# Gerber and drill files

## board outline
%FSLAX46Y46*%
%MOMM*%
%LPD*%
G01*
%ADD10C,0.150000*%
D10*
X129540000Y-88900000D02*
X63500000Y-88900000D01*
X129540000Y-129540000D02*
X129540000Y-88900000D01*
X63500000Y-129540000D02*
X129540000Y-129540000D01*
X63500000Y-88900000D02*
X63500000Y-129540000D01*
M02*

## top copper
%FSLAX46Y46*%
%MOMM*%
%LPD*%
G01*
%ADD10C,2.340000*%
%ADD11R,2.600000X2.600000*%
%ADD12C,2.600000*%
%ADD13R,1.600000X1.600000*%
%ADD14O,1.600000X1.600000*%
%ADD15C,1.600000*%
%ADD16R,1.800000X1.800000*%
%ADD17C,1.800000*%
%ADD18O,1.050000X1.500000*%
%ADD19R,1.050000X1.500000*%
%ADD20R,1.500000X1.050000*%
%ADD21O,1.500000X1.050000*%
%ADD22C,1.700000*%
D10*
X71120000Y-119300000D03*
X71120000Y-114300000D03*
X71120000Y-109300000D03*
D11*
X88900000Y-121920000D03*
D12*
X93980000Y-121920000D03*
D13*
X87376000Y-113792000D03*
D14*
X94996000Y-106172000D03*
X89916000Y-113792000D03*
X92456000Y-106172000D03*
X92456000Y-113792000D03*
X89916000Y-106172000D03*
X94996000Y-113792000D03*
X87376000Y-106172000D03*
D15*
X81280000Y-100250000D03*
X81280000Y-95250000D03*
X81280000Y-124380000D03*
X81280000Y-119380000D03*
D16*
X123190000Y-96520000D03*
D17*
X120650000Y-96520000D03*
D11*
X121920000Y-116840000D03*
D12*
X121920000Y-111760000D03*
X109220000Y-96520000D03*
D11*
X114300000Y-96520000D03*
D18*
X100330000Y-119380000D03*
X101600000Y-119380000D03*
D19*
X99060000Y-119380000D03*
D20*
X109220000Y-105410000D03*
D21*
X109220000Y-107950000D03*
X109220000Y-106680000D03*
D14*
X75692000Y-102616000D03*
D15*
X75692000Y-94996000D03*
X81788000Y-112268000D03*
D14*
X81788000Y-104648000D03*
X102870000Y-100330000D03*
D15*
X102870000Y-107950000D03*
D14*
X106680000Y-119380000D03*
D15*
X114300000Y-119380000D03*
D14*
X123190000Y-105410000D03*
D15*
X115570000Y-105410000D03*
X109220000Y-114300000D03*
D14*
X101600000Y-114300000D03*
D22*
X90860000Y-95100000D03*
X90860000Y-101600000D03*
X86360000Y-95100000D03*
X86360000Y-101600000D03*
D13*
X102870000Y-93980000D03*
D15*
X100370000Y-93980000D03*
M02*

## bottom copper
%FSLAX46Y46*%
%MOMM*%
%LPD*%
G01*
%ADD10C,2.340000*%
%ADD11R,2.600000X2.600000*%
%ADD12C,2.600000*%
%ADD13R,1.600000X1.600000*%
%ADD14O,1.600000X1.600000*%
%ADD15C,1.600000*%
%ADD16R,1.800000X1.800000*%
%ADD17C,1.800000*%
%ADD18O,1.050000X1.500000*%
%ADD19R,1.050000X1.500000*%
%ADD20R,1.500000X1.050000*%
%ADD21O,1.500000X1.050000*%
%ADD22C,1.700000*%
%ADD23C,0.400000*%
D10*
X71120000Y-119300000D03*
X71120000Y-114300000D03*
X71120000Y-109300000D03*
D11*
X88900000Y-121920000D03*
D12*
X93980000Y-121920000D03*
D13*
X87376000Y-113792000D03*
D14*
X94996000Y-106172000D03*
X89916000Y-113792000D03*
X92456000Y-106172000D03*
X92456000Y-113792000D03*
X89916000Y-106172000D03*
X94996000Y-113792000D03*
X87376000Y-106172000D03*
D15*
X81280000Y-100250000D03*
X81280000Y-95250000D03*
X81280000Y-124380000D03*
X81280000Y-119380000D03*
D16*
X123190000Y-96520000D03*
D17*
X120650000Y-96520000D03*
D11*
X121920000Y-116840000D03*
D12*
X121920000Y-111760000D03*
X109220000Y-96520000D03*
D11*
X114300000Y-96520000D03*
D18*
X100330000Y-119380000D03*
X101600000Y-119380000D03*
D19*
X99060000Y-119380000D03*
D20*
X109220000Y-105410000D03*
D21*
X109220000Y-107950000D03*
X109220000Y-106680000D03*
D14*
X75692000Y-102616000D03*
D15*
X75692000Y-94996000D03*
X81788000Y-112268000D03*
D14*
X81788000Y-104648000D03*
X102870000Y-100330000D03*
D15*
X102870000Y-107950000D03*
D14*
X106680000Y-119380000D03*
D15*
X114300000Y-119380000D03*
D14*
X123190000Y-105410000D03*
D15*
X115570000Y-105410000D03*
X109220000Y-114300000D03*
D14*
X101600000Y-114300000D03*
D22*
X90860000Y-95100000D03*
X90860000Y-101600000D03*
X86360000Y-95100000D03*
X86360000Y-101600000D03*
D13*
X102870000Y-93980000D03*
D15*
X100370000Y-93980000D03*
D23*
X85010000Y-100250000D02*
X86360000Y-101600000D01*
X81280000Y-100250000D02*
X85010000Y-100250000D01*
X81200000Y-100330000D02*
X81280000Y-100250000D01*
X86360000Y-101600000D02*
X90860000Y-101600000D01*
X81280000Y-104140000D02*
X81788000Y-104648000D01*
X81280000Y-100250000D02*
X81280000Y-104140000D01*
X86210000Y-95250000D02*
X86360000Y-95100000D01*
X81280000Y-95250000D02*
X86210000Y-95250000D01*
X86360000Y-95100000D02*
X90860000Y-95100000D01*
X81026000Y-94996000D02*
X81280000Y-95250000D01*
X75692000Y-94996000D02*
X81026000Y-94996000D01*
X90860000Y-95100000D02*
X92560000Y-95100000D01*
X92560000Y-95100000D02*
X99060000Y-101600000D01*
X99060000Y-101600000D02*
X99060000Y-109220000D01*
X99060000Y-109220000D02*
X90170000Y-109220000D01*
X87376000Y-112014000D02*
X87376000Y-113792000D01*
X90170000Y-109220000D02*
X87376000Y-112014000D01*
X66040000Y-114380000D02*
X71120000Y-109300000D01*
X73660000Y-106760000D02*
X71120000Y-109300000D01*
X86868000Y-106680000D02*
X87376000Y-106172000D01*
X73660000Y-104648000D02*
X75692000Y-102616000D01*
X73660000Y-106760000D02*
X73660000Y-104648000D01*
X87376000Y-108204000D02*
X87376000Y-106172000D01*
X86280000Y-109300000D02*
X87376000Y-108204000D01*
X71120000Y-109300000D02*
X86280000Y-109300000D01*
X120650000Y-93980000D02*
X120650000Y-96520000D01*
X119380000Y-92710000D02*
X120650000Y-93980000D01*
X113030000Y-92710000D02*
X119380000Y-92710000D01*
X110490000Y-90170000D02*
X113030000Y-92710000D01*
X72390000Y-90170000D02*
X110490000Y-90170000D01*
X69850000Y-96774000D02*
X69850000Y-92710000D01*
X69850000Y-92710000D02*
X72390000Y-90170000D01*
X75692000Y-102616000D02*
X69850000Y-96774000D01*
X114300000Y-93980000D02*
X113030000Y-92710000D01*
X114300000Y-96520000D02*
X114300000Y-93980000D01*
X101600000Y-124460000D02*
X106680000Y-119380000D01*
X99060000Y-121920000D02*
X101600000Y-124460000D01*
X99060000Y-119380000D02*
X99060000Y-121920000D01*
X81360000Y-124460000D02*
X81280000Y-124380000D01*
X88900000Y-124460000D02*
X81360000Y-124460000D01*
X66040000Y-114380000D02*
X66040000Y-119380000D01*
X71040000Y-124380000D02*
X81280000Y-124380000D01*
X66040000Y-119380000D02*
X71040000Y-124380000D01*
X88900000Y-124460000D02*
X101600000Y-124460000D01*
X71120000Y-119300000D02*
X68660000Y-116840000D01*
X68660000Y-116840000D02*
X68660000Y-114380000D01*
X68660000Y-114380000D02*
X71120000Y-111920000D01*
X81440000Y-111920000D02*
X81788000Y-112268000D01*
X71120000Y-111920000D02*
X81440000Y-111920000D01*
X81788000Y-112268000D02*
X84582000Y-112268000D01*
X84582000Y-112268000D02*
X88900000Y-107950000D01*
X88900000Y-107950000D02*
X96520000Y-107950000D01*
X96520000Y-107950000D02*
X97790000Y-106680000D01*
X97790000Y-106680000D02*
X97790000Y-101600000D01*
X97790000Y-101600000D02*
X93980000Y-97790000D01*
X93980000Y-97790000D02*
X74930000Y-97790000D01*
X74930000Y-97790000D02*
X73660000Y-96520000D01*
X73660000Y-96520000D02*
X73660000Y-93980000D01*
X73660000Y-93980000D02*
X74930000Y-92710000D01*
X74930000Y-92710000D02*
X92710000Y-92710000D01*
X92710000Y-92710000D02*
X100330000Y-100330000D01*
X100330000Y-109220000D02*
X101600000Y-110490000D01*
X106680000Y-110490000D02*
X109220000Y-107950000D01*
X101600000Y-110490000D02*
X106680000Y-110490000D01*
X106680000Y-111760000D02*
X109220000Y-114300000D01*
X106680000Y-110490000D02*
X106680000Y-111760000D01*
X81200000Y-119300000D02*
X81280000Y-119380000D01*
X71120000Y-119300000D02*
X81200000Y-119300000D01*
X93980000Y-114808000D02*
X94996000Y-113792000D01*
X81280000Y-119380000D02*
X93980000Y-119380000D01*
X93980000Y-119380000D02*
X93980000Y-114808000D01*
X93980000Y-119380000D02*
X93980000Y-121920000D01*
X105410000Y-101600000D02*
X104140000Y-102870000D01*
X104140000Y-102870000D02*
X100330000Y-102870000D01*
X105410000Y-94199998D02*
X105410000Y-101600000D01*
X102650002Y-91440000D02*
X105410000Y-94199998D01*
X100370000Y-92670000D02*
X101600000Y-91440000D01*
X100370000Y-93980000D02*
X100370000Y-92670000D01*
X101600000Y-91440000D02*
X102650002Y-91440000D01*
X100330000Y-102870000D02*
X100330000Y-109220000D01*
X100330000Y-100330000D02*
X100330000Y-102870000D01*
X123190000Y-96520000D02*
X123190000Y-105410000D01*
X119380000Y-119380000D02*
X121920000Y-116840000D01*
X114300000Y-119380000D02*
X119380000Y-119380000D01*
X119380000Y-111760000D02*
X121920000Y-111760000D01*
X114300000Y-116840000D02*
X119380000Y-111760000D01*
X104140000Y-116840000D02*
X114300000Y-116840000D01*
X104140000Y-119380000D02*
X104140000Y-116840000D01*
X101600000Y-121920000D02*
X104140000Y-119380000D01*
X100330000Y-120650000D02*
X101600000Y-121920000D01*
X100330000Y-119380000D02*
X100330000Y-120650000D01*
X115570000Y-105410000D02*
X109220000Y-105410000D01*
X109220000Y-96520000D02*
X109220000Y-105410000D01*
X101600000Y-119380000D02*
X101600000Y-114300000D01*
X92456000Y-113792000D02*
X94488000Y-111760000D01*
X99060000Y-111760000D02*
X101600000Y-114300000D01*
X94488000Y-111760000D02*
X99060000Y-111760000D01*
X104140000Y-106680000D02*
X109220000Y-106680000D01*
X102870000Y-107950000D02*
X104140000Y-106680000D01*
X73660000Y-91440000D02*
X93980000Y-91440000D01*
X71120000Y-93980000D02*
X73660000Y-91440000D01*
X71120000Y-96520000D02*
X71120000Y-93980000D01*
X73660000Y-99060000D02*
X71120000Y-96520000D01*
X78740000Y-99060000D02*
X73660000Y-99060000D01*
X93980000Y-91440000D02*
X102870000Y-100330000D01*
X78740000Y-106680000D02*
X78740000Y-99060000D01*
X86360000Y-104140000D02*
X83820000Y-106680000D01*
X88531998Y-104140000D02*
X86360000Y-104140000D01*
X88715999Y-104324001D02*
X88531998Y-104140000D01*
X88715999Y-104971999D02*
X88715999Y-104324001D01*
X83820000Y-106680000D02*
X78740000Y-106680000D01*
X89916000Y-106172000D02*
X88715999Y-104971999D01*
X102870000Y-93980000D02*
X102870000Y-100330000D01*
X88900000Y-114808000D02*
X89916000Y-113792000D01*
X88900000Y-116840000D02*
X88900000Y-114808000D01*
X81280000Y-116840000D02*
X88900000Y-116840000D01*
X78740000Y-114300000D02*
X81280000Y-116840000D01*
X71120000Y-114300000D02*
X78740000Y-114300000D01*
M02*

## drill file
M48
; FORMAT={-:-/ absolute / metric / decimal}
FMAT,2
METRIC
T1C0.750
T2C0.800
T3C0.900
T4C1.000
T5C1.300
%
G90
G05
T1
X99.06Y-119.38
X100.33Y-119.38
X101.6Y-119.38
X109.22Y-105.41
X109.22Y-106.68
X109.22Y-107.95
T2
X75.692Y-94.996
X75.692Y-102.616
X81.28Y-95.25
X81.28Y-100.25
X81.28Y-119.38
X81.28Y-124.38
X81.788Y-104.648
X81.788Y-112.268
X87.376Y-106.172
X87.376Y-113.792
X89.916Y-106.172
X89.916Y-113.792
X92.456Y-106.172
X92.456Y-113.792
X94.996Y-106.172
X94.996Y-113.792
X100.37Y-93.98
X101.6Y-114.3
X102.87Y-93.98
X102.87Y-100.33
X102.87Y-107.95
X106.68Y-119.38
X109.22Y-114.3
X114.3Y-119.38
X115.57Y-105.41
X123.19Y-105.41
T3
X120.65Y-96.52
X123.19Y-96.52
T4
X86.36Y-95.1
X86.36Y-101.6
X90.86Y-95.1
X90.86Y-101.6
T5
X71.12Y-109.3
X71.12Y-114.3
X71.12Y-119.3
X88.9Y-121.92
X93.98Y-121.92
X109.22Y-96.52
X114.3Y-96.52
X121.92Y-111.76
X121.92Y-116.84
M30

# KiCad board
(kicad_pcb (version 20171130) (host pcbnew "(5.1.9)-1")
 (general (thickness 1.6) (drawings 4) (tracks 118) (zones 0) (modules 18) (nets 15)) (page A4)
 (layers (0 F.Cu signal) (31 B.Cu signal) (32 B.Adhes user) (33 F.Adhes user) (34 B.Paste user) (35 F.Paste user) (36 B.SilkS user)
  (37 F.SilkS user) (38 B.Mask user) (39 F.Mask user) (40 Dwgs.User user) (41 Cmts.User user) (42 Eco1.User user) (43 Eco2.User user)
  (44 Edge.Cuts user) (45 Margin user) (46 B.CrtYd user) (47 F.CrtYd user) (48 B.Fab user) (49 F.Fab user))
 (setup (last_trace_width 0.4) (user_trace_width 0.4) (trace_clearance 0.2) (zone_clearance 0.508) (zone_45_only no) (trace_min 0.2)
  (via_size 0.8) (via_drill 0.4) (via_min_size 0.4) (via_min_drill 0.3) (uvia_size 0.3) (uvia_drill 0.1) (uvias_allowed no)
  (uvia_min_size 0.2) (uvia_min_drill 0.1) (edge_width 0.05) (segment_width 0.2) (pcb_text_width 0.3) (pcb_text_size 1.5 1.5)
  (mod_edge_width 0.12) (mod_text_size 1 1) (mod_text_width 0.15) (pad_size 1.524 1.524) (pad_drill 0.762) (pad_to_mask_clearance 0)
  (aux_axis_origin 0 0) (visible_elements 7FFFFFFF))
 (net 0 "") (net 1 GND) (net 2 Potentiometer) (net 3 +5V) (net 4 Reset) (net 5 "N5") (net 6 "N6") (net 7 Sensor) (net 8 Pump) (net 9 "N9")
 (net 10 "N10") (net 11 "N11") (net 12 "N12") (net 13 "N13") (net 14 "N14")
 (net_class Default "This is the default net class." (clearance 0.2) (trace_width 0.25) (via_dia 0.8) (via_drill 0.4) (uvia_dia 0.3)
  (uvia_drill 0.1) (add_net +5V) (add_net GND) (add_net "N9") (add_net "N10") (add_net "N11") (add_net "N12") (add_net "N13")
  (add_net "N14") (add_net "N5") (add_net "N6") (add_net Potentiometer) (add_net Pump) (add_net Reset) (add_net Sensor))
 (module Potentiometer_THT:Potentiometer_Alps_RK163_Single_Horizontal (layer F.Cu) (at 71.12 109.3 180)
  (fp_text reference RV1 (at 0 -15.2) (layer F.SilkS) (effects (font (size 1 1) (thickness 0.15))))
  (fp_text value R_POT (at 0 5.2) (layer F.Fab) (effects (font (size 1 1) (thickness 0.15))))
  (pad 3 thru_hole circle (at 0 -10 180) (size 2.34 2.34) (drill 1.3) (layers *.Cu *.Mask) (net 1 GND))
  (pad 2 thru_hole circle (at 0 -5 180) (size 2.34 2.34) (drill 1.3) (layers *.Cu *.Mask) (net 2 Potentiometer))
  (pad 1 thru_hole circle (at 0 0 180) (size 2.34 2.34) (drill 1.3) (layers *.Cu *.Mask) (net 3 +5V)))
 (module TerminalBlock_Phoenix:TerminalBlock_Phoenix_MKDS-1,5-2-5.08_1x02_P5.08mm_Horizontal (layer F.Cu) (at 88.9 121.92)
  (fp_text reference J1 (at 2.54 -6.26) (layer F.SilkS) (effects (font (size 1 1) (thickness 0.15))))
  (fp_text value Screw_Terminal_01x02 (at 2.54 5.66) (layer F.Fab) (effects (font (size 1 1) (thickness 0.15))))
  (pad 1 thru_hole rect (at 0 0) (size 2.6 2.6) (drill 1.3) (layers *.Cu *.Mask) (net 3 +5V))
  (pad 2 thru_hole circle (at 5.08 0) (size 2.6 2.6) (drill 1.3) (layers *.Cu *.Mask) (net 1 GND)))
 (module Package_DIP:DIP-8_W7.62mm (layer F.Cu) (at 87.376 113.792 90)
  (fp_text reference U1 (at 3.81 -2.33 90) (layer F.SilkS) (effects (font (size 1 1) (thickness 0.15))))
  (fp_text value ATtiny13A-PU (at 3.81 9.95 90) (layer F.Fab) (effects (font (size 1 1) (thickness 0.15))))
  (pad 1 thru_hole rect (at 0 0 90) (size 1.6 1.6) (drill 0.8) (layers *.Cu *.Mask) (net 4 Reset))
  (pad 5 thru_hole oval (at 7.62 7.62 90) (size 1.6 1.6) (drill 0.8) (layers *.Cu *.Mask) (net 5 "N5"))
  (pad 2 thru_hole oval (at 0 2.54 90) (size 1.6 1.6) (drill 0.8) (layers *.Cu *.Mask) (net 2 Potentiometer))
  (pad 6 thru_hole oval (at 7.62 5.08 90) (size 1.6 1.6) (drill 0.8) (layers *.Cu *.Mask) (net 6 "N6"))
  (pad 3 thru_hole oval (at 0 5.08 90) (size 1.6 1.6) (drill 0.8) (layers *.Cu *.Mask) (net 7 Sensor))
  (pad 7 thru_hole oval (at 7.62 2.54 90) (size 1.6 1.6) (drill 0.8) (layers *.Cu *.Mask) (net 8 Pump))
  (pad 4 thru_hole oval (at 0 7.62 90) (size 1.6 1.6) (drill 0.8) (layers *.Cu *.Mask) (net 1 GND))
  (pad 8 thru_hole oval (at 7.62 0 90) (size 1.6 1.6) (drill 0.8) (layers *.Cu *.Mask) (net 3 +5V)))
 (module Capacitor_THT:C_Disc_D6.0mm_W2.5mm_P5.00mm (layer F.Cu) (at 81.28 95.25 270)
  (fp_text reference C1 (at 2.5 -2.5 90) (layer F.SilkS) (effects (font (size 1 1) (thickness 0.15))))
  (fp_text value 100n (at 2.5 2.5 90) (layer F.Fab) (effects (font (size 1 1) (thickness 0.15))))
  (pad 2 thru_hole circle (at 5 0 270) (size 1.6 1.6) (drill 0.8) (layers *.Cu *.Mask) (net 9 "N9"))
  (pad 1 thru_hole circle (at 0 0 270) (size 1.6 1.6) (drill 0.8) (layers *.Cu *.Mask) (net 4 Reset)))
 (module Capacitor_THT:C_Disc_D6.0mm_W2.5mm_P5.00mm (layer F.Cu) (at 81.28 124.38 90)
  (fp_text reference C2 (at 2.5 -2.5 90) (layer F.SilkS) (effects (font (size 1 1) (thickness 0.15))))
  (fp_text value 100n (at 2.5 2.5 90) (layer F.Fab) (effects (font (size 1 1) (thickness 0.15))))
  (pad 1 thru_hole circle (at 0 0 90) (size 1.6 1.6) (drill 0.8) (layers *.Cu *.Mask) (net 3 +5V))
  (pad 2 thru_hole circle (at 5 0 90) (size 1.6 1.6) (drill 0.8) (layers *.Cu *.Mask) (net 1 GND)))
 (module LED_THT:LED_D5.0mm (layer F.Cu) (at 123.19 96.52 180)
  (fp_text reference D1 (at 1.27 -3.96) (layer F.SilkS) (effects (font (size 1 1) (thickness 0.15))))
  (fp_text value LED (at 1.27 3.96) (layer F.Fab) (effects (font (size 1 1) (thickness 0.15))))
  (pad 1 thru_hole rect (at 0 0 180) (size 1.8 1.8) (drill 0.9) (layers *.Cu *.Mask) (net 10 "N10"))
  (pad 2 thru_hole circle (at 2.54 0 180) (size 1.8 1.8) (drill 0.9) (layers *.Cu *.Mask) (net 3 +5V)))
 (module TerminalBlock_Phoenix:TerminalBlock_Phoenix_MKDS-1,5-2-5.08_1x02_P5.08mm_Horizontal (layer F.Cu) (at 121.92 116.84 90)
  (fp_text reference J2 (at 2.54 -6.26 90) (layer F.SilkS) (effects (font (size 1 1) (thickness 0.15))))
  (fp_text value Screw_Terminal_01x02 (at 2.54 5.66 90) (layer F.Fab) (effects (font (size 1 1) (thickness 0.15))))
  (pad 1 thru_hole rect (at 0 0 90) (size 2.6 2.6) (drill 1.3) (layers *.Cu *.Mask) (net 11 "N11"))
  (pad 2 thru_hole circle (at 5.08 0 90) (size 2.6 2.6) (drill 1.3) (layers *.Cu *.Mask) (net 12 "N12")))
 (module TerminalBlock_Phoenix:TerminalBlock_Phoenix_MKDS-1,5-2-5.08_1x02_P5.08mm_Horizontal (layer F.Cu) (at 114.3 96.52 180)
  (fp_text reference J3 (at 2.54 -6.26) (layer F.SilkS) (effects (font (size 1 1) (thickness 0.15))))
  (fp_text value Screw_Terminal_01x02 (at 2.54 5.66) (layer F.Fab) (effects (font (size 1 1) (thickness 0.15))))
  (pad 2 thru_hole circle (at 5.08 0 180) (size 2.6 2.6) (drill 1.3) (layers *.Cu *.Mask) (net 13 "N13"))
  (pad 1 thru_hole rect (at 0 0 180) (size 2.6 2.6) (drill 1.3) (layers *.Cu *.Mask) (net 3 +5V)))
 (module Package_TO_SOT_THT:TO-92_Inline (layer F.Cu) (at 99.06 119.38)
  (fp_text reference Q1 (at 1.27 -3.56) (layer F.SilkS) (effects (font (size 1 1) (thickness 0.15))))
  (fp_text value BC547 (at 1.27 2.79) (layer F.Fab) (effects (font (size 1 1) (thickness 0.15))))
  (pad 2 thru_hole oval (at 1.27 0) (size 1.05 1.5) (drill 0.75) (layers *.Cu *.Mask) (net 12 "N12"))
  (pad 3 thru_hole oval (at 2.54 0) (size 1.05 1.5) (drill 0.75) (layers *.Cu *.Mask) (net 7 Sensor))
  (pad 1 thru_hole rect (at 0 0) (size 1.05 1.5) (drill 0.75) (layers *.Cu *.Mask) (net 3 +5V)))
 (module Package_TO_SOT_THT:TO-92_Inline (layer F.Cu) (at 109.22 105.41 270)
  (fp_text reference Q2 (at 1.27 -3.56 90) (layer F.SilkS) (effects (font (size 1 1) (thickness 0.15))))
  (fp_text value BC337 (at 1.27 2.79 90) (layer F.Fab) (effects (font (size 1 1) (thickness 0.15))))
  (pad 1 thru_hole rect (at 0 0 270) (size 1.05 1.5) (drill 0.75) (layers *.Cu *.Mask) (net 13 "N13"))
  (pad 3 thru_hole oval (at 2.54 0 270) (size 1.05 1.5) (drill 0.75) (layers *.Cu *.Mask) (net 1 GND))
  (pad 2 thru_hole oval (at 1.27 0 270) (size 1.05 1.5) (drill 0.75) (layers *.Cu *.Mask) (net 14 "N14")))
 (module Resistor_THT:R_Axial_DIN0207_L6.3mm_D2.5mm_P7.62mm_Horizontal (layer F.Cu) (at 75.692 94.996 270)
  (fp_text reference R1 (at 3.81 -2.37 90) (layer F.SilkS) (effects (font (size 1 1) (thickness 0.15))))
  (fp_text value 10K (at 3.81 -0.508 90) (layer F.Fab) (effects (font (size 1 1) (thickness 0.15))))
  (pad 2 thru_hole oval (at 7.62 0 270) (size 1.6 1.6) (drill 0.8) (layers *.Cu *.Mask) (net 3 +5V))
  (pad 1 thru_hole circle (at 0 0 270) (size 1.6 1.6) (drill 0.8) (layers *.Cu *.Mask) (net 4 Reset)))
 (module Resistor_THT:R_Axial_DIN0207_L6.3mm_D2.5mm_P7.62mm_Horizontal (layer F.Cu) (at 81.788 112.268 90)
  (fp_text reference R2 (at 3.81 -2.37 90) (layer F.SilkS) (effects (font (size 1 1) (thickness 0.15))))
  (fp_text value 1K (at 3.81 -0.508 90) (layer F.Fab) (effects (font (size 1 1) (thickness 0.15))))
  (pad 1 thru_hole circle (at 0 0 90) (size 1.6 1.6) (drill 0.8) (layers *.Cu *.Mask) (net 1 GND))
  (pad 2 thru_hole oval (at 7.62 0 90) (size 1.6 1.6) (drill 0.8) (layers *.Cu *.Mask) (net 9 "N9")))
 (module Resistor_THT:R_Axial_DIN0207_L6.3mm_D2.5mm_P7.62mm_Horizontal (layer F.Cu) (at 102.87 107.95 90)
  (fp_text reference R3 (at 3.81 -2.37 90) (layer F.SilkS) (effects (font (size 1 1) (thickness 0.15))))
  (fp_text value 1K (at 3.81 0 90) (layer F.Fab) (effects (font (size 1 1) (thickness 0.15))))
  (pad 2 thru_hole oval (at 7.62 0 90) (size 1.6 1.6) (drill 0.8) (layers *.Cu *.Mask) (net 8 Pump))
  (pad 1 thru_hole circle (at 0 0 90) (size 1.6 1.6) (drill 0.8) (layers *.Cu *.Mask) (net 14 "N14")))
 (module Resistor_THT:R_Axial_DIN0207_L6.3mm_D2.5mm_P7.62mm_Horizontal (layer F.Cu) (at 114.3 119.38 180)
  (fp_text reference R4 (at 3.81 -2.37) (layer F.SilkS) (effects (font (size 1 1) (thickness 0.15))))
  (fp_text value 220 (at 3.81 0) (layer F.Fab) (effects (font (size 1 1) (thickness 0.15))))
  (pad 2 thru_hole oval (at 7.62 0 180) (size 1.6 1.6) (drill 0.8) (layers *.Cu *.Mask) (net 3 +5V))
  (pad 1 thru_hole circle (at 0 0 180) (size 1.6 1.6) (drill 0.8) (layers *.Cu *.Mask) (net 11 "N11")))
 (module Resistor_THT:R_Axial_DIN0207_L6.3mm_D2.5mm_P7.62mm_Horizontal (layer F.Cu) (at 115.57 105.41)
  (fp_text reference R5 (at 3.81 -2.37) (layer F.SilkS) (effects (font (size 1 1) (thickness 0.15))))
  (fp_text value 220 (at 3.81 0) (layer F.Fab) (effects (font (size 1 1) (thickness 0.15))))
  (pad 2 thru_hole oval (at 7.62 0) (size 1.6 1.6) (drill 0.8) (layers *.Cu *.Mask) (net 10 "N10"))
  (pad 1 thru_hole circle (at 0 0) (size 1.6 1.6) (drill 0.8) (layers *.Cu *.Mask) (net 13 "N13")))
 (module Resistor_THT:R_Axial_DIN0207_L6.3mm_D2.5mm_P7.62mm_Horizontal (layer F.Cu) (at 109.22 114.3 180)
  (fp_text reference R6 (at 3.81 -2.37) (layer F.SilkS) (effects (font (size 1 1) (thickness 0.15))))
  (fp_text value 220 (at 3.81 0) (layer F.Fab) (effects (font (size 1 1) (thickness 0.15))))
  (pad 1 thru_hole circle (at 0 0 180) (size 1.6 1.6) (drill 0.8) (layers *.Cu *.Mask) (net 1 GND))
  (pad 2 thru_hole oval (at 7.62 0 180) (size 1.6 1.6) (drill 0.8) (layers *.Cu *.Mask) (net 7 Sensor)))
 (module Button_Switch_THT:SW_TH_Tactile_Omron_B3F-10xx (layer F.Cu) (at 86.36 101.6 90)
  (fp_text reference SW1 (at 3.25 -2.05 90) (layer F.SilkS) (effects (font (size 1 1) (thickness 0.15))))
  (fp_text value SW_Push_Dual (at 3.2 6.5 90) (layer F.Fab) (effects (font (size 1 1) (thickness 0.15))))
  (pad 4 thru_hole circle (at 6.5 4.5 90) (size 1.7 1.7) (drill 1) (layers *.Cu *.Mask) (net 4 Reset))
  (pad 3 thru_hole circle (at 0 4.5 90) (size 1.7 1.7) (drill 1) (layers *.Cu *.Mask) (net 9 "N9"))
  (pad 2 thru_hole circle (at 6.5 0 90) (size 1.7 1.7) (drill 1) (layers *.Cu *.Mask) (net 4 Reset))
  (pad 1 thru_hole circle (at 0 0 90) (size 1.7 1.7) (drill 1) (layers *.Cu *.Mask) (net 9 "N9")))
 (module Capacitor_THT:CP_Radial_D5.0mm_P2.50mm (layer F.Cu) (at 102.87 93.98 180)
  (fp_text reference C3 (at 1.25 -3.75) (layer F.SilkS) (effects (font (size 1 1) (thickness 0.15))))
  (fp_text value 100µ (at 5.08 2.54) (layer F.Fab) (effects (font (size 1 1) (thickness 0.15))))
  (pad 1 thru_hole rect (at 0 0 180) (size 1.6 1.6) (drill 0.8) (layers *.Cu *.Mask) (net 8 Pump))
  (pad 2 thru_hole circle (at 2.5 0 180) (size 1.6 1.6) (drill 0.8) (layers *.Cu *.Mask) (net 1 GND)))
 (gr_line (start 129.54 88.9) (end 63.5 88.9) (layer Edge.Cuts) (width 0.15))
 (gr_line (start 129.54 129.54) (end 129.54 88.9) (layer Edge.Cuts) (width 0.15))
 (gr_line (start 63.5 129.54) (end 129.54 129.54) (layer Edge.Cuts) (width 0.15))
 (gr_line (start 63.5 88.9) (end 63.5 129.54) (layer Edge.Cuts) (width 0.15))
 (segment (start 85.01 100.25) (end 86.36 101.6) (width 0.4) (layer B.Cu) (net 9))
 (segment (start 81.28 100.25) (end 85.01 100.25) (width 0.4) (layer B.Cu) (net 9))
 (segment (start 81.2 100.33) (end 81.28 100.25) (width 0.4) (layer B.Cu) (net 9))
 (segment (start 86.36 101.6) (end 90.86 101.6) (width 0.4) (layer B.Cu) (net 9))
 (segment (start 81.28 104.14) (end 81.788 104.648) (width 0.4) (layer B.Cu) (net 9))
 (segment (start 81.28 100.25) (end 81.28 104.14) (width 0.4) (layer B.Cu) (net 9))
 (segment (start 86.21 95.25) (end 86.36 95.1) (width 0.4) (layer B.Cu) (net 4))
 (segment (start 81.28 95.25) (end 86.21 95.25) (width 0.4) (layer B.Cu) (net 4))
 (segment (start 86.36 95.1) (end 90.86 95.1) (width 0.4) (layer B.Cu) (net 4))
 (segment (start 81.026 94.996) (end 81.28 95.25) (width 0.4) (layer B.Cu) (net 4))
 (segment (start 75.692 94.996) (end 81.026 94.996) (width 0.4) (layer B.Cu) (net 4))
 (segment (start 90.86 95.1) (end 92.56 95.1) (width 0.4) (layer B.Cu) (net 4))
 (segment (start 92.56 95.1) (end 99.06 101.6) (width 0.4) (layer B.Cu) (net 4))
 (segment (start 99.06 101.6) (end 99.06 109.22) (width 0.4) (layer B.Cu) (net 4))
 (segment (start 99.06 109.22) (end 90.17 109.22) (width 0.4) (layer B.Cu) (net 4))
 (segment (start 87.376 112.014) (end 87.376 113.792) (width 0.4) (layer B.Cu) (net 4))
 (segment (start 90.17 109.22) (end 87.376 112.014) (width 0.4) (layer B.Cu) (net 4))
 (segment (start 66.04 114.38) (end 71.12 109.3) (width 0.4) (layer B.Cu) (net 3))
 (segment (start 73.66 106.76) (end 71.12 109.3) (width 0.4) (layer B.Cu) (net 3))
 (segment (start 86.868 106.68) (end 87.376 106.172) (width 0.4) (layer B.Cu) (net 3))
 (segment (start 73.66 104.648) (end 75.692 102.616) (width 0.4) (layer B.Cu) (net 3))
 (segment (start 73.66 106.76) (end 73.66 104.648) (width 0.4) (layer B.Cu) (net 3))
 (segment (start 87.376 108.204) (end 87.376 106.172) (width 0.4) (layer B.Cu) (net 3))
 (segment (start 86.28 109.3) (end 87.376 108.204) (width 0.4) (layer B.Cu) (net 3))
 (segment (start 71.12 109.3) (end 86.28 109.3) (width 0.4) (layer B.Cu) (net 3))
 (segment (start 120.65 93.98) (end 120.65 96.52) (width 0.4) (layer B.Cu) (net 3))
 (segment (start 119.38 92.71) (end 120.65 93.98) (width 0.4) (layer B.Cu) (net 3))
 (segment (start 113.03 92.71) (end 119.38 92.71) (width 0.4) (layer B.Cu) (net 3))
 (segment (start 110.49 90.17) (end 113.03 92.71) (width 0.4) (layer B.Cu) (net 3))
 (segment (start 72.39 90.17) (end 110.49 90.17) (width 0.4) (layer B.Cu) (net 3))
 (segment (start 69.85 96.774) (end 69.85 92.71) (width 0.4) (layer B.Cu) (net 3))
 (segment (start 69.85 92.71) (end 72.39 90.17) (width 0.4) (layer B.Cu) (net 3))
 (segment (start 75.692 102.616) (end 69.85 96.774) (width 0.4) (layer B.Cu) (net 3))
 (segment (start 114.3 93.98) (end 113.03 92.71) (width 0.4) (layer B.Cu) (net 3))
 (segment (start 114.3 96.52) (end 114.3 93.98) (width 0.4) (layer B.Cu) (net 3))
 (segment (start 101.6 124.46) (end 106.68 119.38) (width 0.4) (layer B.Cu) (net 3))
 (segment (start 99.06 121.92) (end 101.6 124.46) (width 0.4) (layer B.Cu) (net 3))
 (segment (start 99.06 119.38) (end 99.06 121.92) (width 0.4) (layer B.Cu) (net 3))
 (segment (start 81.36 124.46) (end 81.28 124.38) (width 0.4) (layer B.Cu) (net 3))
 (segment (start 88.9 124.46) (end 81.36 124.46) (width 0.4) (layer B.Cu) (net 3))
 (segment (start 66.04 114.38) (end 66.04 119.38) (width 0.4) (layer B.Cu) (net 3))
 (segment (start 71.04 124.38) (end 81.28 124.38) (width 0.4) (layer B.Cu) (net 3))
 (segment (start 66.04 119.38) (end 71.04 124.38) (width 0.4) (layer B.Cu) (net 3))
 (segment (start 88.9 124.46) (end 101.6 124.46) (width 0.4) (layer B.Cu) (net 3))
 (segment (start 71.12 119.3) (end 68.66 116.84) (width 0.4) (layer B.Cu) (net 1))
 (segment (start 68.66 116.84) (end 68.66 114.38) (width 0.4) (layer B.Cu) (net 1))
 (segment (start 68.66 114.38) (end 71.12 111.92) (width 0.4) (layer B.Cu) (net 1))
 (segment (start 81.44 111.92) (end 81.788 112.268) (width 0.4) (layer B.Cu) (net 1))
 (segment (start 71.12 111.92) (end 81.44 111.92) (width 0.4) (layer B.Cu) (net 1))
 (segment (start 81.788 112.268) (end 84.582 112.268) (width 0.4) (layer B.Cu) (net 1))
 (segment (start 84.582 112.268) (end 88.9 107.95) (width 0.4) (layer B.Cu) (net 1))
 (segment (start 88.9 107.95) (end 96.52 107.95) (width 0.4) (layer B.Cu) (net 1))
 (segment (start 96.52 107.95) (end 97.79 106.68) (width 0.4) (layer B.Cu) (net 1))
 (segment (start 97.79 106.68) (end 97.79 101.6) (width 0.4) (layer B.Cu) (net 1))
 (segment (start 97.79 101.6) (end 93.98 97.79) (width 0.4) (layer B.Cu) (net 1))
 (segment (start 93.98 97.79) (end 74.93 97.79) (width 0.4) (layer B.Cu) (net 1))
 (segment (start 74.93 97.79) (end 73.66 96.52) (width 0.4) (layer B.Cu) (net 1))
 (segment (start 73.66 96.52) (end 73.66 93.98) (width 0.4) (layer B.Cu) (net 1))
 (segment (start 73.66 93.98) (end 74.93 92.71) (width 0.4) (layer B.Cu) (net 1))
 (segment (start 74.93 92.71) (end 92.71 92.71) (width 0.4) (layer B.Cu) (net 1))
 (segment (start 92.71 92.71) (end 100.33 100.33) (width 0.4) (layer B.Cu) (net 1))
 (segment (start 100.33 109.22) (end 101.6 110.49) (width 0.4) (layer B.Cu) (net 1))
 (segment (start 106.68 110.49) (end 109.22 107.95) (width 0.4) (layer B.Cu) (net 1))
 (segment (start 101.6 110.49) (end 106.68 110.49) (width 0.4) (layer B.Cu) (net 1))
 (segment (start 106.68 111.76) (end 109.22 114.3) (width 0.4) (layer B.Cu) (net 1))
 (segment (start 106.68 110.49) (end 106.68 111.76) (width 0.4) (layer B.Cu) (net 1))
 (segment (start 81.2 119.3) (end 81.28 119.38) (width 0.4) (layer B.Cu) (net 1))
 (segment (start 71.12 119.3) (end 81.2 119.3) (width 0.4) (layer B.Cu) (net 1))
 (segment (start 93.98 114.808) (end 94.996 113.792) (width 0.4) (layer B.Cu) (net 1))
 (segment (start 81.28 119.38) (end 93.98 119.38) (width 0.4) (layer B.Cu) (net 1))
 (segment (start 93.98 119.38) (end 93.98 114.808) (width 0.4) (layer B.Cu) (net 1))
 (segment (start 93.98 119.38) (end 93.98 121.92) (width 0.4) (layer B.Cu) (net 1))
 (segment (start 105.41 101.6) (end 104.14 102.87) (width 0.4) (layer B.Cu) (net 1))
 (segment (start 104.14 102.87) (end 100.33 102.87) (width 0.4) (layer B.Cu) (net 1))
 (segment (start 105.41 94.199998) (end 105.41 101.6) (width 0.4) (layer B.Cu) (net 1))
 (segment (start 102.650002 91.44) (end 105.41 94.199998) (width 0.4) (layer B.Cu) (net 1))
 (segment (start 100.37 92.67) (end 101.6 91.44) (width 0.4) (layer B.Cu) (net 1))
 (segment (start 100.37 93.98) (end 100.37 92.67) (width 0.4) (layer B.Cu) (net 1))
 (segment (start 101.6 91.44) (end 102.650002 91.44) (width 0.4) (layer B.Cu) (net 1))
 (segment (start 100.33 102.87) (end 100.33 109.22) (width 0.4) (layer B.Cu) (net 1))
 (segment (start 100.33 100.33) (end 100.33 102.87) (width 0.4) (layer B.Cu) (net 1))
 (segment (start 123.19 96.52) (end 123.19 105.41) (width 0.4) (layer B.Cu) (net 10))
 (segment (start 119.38 119.38) (end 121.92 116.84) (width 0.4) (layer B.Cu) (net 11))
 (segment (start 114.3 119.38) (end 119.38 119.38) (width 0.4) (layer B.Cu) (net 11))
 (segment (start 119.38 111.76) (end 121.92 111.76) (width 0.4) (layer B.Cu) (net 12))
 (segment (start 114.3 116.84) (end 119.38 111.76) (width 0.4) (layer B.Cu) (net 12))
 (segment (start 104.14 116.84) (end 114.3 116.84) (width 0.4) (layer B.Cu) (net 12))
 (segment (start 104.14 119.38) (end 104.14 116.84) (width 0.4) (layer B.Cu) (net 12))
 (segment (start 101.6 121.92) (end 104.14 119.38) (width 0.4) (layer B.Cu) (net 12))
 (segment (start 100.33 120.65) (end 101.6 121.92) (width 0.4) (layer B.Cu) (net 12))
 (segment (start 100.33 119.38) (end 100.33 120.65) (width 0.4) (layer B.Cu) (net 12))
 (segment (start 115.57 105.41) (end 109.22 105.41) (width 0.4) (layer B.Cu) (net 13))
 (segment (start 109.22 96.52) (end 109.22 105.41) (width 0.4) (layer B.Cu) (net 13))
 (segment (start 101.6 119.38) (end 101.6 114.3) (width 0.4) (layer B.Cu) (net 7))
 (segment (start 92.456 113.792) (end 94.488 111.76) (width 0.4) (layer B.Cu) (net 7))
 (segment (start 99.06 111.76) (end 101.6 114.3) (width 0.4) (layer B.Cu) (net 7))
 (segment (start 94.488 111.76) (end 99.06 111.76) (width 0.4) (layer B.Cu) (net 7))
 (segment (start 104.14 106.68) (end 109.22 106.68) (width 0.4) (layer B.Cu) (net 14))
 (segment (start 102.87 107.95) (end 104.14 106.68) (width 0.4) (layer B.Cu) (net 14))
 (segment (start 73.66 91.44) (end 93.98 91.44) (width 0.4) (layer B.Cu) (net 8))
 (segment (start 71.12 93.98) (end 73.66 91.44) (width 0.4) (layer B.Cu) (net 8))
 (segment (start 71.12 96.52) (end 71.12 93.98) (width 0.4) (layer B.Cu) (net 8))
 (segment (start 73.66 99.06) (end 71.12 96.52) (width 0.4) (layer B.Cu) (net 8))
 (segment (start 78.74 99.06) (end 73.66 99.06) (width 0.4) (layer B.Cu) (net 8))
 (segment (start 93.98 91.44) (end 102.87 100.33) (width 0.4) (layer B.Cu) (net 8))
 (segment (start 78.74 106.68) (end 78.74 99.06) (width 0.4) (layer B.Cu) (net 8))
 (segment (start 86.36 104.14) (end 83.82 106.68) (width 0.4) (layer B.Cu) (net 8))
 (segment (start 88.531998 104.14) (end 86.36 104.14) (width 0.4) (layer B.Cu) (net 8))
 (segment (start 88.715999 104.324001) (end 88.531998 104.14) (width 0.4) (layer B.Cu) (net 8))
 (segment (start 88.715999 104.971999) (end 88.715999 104.324001) (width 0.4) (layer B.Cu) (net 8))
 (segment (start 83.82 106.68) (end 78.74 106.68) (width 0.4) (layer B.Cu) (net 8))
 (segment (start 89.916 106.172) (end 88.715999 104.971999) (width 0.4) (layer B.Cu) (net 8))
 (segment (start 102.87 93.98) (end 102.87 100.33) (width 0.4) (layer B.Cu) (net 8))
 (segment (start 88.9 114.808) (end 89.916 113.792) (width 0.4) (layer B.Cu) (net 2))
 (segment (start 88.9 116.84) (end 88.9 114.808) (width 0.4) (layer B.Cu) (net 2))
 (segment (start 81.28 116.84) (end 88.9 116.84) (width 0.4) (layer B.Cu) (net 2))
 (segment (start 78.74 114.3) (end 81.28 116.84) (width 0.4) (layer B.Cu) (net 2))
 (segment (start 71.12 114.3) (end 78.74 114.3) (width 0.4) (layer B.Cu) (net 2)))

